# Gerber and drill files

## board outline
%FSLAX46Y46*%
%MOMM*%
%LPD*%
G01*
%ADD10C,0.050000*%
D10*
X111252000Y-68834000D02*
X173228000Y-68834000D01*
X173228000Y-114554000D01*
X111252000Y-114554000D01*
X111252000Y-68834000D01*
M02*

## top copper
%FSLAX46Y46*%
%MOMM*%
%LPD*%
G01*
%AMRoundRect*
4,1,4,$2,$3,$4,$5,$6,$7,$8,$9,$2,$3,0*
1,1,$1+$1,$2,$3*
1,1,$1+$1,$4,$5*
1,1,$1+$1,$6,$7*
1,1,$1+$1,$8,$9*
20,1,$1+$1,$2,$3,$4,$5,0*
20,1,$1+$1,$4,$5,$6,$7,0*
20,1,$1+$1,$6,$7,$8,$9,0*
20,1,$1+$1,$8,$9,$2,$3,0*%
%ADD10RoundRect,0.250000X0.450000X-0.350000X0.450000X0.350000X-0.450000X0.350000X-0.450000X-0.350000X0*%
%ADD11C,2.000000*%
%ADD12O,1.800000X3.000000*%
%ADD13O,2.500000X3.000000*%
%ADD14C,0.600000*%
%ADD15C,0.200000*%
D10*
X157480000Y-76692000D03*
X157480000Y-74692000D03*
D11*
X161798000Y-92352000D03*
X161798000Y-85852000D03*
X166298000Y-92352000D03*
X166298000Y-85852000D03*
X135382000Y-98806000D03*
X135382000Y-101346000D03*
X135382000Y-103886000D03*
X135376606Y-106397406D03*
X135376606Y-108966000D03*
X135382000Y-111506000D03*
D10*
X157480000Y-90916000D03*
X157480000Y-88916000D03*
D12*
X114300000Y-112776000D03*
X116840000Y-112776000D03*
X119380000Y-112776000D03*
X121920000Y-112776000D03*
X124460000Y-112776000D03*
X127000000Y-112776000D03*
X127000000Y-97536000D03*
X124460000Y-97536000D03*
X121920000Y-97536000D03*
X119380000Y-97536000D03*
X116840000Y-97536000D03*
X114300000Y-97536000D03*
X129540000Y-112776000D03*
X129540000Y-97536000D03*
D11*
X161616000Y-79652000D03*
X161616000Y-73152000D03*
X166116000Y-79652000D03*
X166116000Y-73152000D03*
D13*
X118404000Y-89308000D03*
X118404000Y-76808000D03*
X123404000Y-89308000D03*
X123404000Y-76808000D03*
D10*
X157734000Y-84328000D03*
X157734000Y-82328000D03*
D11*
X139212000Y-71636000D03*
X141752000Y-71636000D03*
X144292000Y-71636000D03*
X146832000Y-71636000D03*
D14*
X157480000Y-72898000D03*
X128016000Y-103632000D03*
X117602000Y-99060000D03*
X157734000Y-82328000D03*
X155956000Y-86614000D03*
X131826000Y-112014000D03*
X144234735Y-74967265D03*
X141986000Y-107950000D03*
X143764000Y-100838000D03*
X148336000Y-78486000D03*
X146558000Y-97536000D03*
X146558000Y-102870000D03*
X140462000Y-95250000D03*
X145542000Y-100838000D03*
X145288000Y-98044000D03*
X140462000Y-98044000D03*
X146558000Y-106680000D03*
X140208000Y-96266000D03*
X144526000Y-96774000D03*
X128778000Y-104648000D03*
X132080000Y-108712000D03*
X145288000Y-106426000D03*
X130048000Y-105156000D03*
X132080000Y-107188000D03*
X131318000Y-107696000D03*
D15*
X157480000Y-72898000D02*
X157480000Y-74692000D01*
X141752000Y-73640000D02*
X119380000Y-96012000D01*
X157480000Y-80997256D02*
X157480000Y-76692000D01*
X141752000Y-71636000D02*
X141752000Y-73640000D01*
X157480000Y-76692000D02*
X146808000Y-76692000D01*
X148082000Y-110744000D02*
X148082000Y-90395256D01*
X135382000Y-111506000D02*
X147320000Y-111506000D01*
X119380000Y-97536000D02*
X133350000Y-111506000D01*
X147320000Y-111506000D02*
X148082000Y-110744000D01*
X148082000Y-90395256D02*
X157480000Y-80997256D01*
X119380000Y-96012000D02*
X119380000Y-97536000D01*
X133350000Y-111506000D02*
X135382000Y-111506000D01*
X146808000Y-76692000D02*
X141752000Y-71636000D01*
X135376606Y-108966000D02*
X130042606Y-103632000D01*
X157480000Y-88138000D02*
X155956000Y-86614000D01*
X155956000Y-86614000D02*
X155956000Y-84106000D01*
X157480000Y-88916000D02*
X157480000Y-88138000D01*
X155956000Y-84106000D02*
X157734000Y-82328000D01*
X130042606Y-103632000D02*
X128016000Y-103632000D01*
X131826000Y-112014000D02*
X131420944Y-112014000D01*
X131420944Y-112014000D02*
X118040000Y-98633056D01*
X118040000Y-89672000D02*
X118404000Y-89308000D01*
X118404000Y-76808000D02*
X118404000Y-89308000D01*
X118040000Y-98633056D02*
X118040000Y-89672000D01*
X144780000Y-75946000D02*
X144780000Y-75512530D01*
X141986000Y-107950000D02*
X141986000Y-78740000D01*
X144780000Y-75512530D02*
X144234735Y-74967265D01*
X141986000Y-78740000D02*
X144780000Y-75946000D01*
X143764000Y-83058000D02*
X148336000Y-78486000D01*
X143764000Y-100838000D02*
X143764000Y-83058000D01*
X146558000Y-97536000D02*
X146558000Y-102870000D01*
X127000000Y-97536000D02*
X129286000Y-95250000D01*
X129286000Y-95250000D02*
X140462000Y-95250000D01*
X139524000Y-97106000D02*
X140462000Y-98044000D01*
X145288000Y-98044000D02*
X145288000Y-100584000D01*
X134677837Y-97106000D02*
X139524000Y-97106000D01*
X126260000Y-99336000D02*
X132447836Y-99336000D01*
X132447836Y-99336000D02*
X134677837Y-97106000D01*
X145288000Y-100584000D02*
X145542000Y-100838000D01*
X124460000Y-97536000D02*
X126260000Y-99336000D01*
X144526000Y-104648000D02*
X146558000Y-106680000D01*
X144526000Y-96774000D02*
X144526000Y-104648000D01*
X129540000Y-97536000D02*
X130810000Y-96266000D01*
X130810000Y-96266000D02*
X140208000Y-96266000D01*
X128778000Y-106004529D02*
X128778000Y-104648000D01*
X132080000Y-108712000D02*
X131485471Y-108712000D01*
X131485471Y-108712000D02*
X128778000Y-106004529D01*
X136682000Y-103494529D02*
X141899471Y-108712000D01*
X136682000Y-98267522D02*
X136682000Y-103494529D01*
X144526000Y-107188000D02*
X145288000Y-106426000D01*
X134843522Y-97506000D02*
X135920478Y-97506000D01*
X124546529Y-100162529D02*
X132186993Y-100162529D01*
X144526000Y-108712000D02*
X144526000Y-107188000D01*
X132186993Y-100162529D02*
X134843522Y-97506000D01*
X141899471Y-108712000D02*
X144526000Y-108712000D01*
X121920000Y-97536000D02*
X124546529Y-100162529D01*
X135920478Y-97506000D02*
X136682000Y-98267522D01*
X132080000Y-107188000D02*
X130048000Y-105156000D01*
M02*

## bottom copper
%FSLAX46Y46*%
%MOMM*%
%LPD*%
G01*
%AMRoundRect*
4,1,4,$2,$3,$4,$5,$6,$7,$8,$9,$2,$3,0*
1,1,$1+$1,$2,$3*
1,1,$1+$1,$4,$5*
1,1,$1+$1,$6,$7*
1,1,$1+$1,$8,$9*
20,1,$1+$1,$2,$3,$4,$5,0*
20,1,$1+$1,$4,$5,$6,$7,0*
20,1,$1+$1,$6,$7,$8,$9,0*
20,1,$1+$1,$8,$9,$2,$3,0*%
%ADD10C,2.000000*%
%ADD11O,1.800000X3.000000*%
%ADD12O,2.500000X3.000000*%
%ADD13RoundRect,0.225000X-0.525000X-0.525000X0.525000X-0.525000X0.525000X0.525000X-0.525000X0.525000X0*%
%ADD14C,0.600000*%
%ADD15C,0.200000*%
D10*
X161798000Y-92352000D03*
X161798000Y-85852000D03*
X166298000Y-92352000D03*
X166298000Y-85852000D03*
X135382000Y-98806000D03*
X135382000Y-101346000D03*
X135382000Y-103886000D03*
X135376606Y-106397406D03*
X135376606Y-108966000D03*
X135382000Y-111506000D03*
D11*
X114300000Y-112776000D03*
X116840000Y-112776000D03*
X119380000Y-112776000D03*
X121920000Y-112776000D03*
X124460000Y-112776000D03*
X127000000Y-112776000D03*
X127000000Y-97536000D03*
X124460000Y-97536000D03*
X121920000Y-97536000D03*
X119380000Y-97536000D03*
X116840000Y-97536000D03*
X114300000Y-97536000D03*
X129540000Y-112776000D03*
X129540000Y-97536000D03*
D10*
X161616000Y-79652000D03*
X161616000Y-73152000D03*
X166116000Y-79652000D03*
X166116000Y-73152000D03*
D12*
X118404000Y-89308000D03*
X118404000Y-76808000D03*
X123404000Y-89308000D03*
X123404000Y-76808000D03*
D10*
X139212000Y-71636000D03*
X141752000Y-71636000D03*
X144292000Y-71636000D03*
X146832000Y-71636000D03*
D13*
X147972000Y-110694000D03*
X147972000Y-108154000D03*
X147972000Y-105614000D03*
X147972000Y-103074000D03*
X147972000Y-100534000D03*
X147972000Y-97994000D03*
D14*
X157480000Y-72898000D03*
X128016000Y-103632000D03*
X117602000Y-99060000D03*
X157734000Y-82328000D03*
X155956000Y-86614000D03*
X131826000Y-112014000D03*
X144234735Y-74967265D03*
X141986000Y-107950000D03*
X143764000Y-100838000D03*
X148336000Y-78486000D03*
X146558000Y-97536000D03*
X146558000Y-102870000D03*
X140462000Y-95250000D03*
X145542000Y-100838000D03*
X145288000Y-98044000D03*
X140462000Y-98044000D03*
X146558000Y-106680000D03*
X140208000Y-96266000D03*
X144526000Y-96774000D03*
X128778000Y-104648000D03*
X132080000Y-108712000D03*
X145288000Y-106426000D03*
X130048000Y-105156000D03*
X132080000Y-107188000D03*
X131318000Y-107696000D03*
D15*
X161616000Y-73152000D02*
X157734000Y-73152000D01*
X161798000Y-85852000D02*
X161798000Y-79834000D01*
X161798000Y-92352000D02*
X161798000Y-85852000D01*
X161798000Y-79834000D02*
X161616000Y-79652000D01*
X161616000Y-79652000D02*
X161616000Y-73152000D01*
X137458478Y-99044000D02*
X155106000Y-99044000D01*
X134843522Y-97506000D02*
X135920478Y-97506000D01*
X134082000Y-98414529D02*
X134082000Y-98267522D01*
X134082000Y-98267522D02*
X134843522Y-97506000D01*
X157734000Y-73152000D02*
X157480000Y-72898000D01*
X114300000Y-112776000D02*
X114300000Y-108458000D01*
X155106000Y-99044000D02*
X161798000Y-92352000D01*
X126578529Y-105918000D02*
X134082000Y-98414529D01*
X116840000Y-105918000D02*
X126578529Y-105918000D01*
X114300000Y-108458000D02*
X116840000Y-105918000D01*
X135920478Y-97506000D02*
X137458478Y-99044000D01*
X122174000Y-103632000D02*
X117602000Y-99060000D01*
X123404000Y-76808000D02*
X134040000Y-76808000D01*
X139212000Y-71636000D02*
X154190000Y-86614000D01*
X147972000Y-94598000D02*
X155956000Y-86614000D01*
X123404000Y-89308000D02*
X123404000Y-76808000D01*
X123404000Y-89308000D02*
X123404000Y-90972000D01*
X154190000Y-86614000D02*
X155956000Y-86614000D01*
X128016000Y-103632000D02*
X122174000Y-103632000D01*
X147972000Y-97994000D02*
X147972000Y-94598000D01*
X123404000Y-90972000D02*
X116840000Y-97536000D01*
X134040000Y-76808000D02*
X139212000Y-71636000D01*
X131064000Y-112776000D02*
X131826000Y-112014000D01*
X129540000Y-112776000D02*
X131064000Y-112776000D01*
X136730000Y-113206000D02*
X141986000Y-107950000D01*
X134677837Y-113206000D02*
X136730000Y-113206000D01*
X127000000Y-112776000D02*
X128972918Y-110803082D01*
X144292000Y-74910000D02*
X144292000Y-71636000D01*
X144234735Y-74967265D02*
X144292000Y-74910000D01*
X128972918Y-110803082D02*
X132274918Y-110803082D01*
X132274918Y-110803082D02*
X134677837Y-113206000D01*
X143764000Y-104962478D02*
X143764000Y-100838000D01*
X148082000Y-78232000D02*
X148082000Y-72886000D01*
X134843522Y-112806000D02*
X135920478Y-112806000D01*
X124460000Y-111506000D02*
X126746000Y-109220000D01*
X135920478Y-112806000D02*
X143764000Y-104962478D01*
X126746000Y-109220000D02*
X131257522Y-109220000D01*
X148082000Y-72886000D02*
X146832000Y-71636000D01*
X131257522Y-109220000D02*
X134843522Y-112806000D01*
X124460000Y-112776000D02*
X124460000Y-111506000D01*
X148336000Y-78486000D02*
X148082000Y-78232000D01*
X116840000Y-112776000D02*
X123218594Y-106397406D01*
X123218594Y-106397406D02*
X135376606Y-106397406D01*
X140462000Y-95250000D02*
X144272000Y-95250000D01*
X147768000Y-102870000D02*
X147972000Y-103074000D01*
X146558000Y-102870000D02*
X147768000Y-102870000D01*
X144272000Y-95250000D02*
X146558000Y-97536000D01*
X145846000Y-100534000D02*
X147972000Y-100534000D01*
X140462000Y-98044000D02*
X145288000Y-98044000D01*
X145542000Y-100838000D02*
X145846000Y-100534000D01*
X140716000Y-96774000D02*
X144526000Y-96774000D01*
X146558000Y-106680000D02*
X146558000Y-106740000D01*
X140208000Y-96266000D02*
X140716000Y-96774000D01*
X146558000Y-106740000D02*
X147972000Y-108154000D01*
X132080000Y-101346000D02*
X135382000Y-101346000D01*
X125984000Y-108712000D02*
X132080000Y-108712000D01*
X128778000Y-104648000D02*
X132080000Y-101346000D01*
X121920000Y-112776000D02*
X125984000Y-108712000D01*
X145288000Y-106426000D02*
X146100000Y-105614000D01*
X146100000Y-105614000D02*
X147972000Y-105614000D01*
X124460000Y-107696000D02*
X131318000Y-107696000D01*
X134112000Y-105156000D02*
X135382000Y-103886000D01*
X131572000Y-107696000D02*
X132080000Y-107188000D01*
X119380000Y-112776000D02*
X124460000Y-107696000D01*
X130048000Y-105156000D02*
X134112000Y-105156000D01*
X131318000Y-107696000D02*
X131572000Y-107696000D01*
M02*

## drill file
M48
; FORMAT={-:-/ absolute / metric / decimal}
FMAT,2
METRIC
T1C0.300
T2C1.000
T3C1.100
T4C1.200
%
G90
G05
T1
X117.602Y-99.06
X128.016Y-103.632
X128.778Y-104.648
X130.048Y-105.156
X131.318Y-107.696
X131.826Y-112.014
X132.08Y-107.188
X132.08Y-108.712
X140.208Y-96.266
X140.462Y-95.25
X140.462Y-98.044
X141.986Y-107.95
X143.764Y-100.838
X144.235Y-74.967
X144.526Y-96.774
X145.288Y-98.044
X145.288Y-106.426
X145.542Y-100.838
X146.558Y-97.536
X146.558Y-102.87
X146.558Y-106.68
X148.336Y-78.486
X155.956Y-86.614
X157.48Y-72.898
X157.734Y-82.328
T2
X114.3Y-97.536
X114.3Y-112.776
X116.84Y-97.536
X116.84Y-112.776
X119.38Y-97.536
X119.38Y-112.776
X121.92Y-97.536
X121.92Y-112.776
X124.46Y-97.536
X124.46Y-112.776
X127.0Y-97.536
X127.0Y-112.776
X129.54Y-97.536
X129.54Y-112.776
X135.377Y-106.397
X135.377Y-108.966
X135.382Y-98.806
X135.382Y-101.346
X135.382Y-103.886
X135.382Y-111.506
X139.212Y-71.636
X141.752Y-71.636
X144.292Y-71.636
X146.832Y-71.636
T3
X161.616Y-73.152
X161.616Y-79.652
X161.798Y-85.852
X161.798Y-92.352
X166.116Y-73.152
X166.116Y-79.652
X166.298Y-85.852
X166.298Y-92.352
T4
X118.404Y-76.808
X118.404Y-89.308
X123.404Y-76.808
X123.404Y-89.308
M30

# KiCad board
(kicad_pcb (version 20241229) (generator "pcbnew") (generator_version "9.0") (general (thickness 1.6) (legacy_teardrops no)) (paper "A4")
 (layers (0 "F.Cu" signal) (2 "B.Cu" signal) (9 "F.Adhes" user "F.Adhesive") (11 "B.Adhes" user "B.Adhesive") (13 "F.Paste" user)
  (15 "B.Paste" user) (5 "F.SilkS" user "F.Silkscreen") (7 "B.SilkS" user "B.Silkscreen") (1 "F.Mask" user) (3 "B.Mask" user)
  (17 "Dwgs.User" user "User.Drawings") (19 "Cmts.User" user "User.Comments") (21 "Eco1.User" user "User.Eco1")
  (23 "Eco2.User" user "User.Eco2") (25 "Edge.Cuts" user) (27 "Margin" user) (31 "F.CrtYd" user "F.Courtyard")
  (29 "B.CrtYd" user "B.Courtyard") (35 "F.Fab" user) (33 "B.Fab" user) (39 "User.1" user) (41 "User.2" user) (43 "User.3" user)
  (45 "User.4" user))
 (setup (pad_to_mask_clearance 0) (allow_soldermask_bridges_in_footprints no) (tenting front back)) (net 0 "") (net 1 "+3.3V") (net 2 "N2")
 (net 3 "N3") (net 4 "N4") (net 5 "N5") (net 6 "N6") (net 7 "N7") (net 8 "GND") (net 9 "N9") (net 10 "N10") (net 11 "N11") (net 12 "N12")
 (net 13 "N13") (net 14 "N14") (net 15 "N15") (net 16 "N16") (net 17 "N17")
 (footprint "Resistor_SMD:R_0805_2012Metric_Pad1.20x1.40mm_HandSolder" (layer "F.Cu") (at 157.48 75.692 90)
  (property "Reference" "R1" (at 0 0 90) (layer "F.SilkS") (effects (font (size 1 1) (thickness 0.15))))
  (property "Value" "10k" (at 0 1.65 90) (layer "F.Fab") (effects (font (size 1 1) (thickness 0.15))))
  (pad "1" smd roundrect (at -1 0 90) (size 1.2 1.4) (layers "F.Cu" "F.Mask" "F.Paste") (roundrect_rratio 0.208333) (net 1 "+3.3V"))
  (pad "2" smd roundrect (at 1 0 90) (size 1.2 1.4) (layers "F.Cu" "F.Mask" "F.Paste") (roundrect_rratio 0.208333) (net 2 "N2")))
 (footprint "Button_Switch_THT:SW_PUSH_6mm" (layer "F.Cu") (at 161.798 92.352 90)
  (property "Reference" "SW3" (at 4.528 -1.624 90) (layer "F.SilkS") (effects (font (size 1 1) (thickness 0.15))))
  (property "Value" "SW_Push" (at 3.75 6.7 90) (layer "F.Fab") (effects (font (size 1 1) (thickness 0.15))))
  (pad "1" thru_hole circle (at 0 0 180) (size 2 2) (drill 1.1) (layers "*.Cu" "*.Mask") (remove_unused_layers no) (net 2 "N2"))
  (pad "1" thru_hole circle (at 6.5 0 180) (size 2 2) (drill 1.1) (layers "*.Cu" "*.Mask") (remove_unused_layers no) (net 2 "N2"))
  (pad "2" thru_hole circle (at 0 4.5 180) (size 2 2) (drill 1.1) (layers "*.Cu" "*.Mask") (remove_unused_layers no) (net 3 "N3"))
  (pad "2" thru_hole circle (at 6.5 4.5 180) (size 2 2) (drill 1.1) (layers "*.Cu" "*.Mask") (remove_unused_layers no) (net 3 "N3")))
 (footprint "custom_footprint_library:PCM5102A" (layer "F.Cu") (at 148.082 103.886)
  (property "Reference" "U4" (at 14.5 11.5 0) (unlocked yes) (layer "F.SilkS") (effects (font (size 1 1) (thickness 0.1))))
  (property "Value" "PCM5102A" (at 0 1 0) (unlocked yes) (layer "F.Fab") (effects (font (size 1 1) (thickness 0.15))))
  (pad "1" thru_hole circle (at -12.7 -5.08) (size 2 2) (drill 1) (layers "*.Cu" "*.Mask") (remove_unused_layers no) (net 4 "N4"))
  (pad "2" thru_hole circle (at -12.7 -2.54) (size 2 2) (drill 1) (layers "*.Cu" "*.Mask") (remove_unused_layers no) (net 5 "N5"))
  (pad "3" thru_hole circle (at -12.7 0) (size 2 2) (drill 1) (layers "*.Cu" "*.Mask") (remove_unused_layers no) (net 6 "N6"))
  (pad "4" thru_hole circle (at -12.705394 2.511406) (size 2 2) (drill 1) (layers "*.Cu" "*.Mask") (remove_unused_layers no) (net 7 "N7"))
  (pad "5" thru_hole circle (at -12.705394 5.08) (size 2 2) (drill 1) (layers "*.Cu" "*.Mask") (remove_unused_layers no) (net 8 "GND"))
  (pad "6" thru_hole circle (at -12.7 7.62) (size 2 2) (drill 1) (layers "*.Cu" "*.Mask") (remove_unused_layers no) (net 1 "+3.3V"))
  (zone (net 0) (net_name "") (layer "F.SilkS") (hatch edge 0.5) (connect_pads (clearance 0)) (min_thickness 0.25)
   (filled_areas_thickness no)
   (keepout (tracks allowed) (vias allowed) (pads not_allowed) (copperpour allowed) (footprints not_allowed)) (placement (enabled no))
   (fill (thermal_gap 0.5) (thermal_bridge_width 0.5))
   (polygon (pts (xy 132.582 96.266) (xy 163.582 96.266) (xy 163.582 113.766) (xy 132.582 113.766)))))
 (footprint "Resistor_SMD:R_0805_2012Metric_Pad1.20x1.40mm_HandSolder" (layer "F.Cu") (at 157.48 89.916 90)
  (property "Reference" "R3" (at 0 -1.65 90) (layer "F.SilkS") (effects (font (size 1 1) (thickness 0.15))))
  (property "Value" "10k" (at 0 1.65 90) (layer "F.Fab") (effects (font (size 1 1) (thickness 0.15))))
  (pad "1" smd roundrect (at -1 0 90) (size 1.2 1.4) (layers "F.Cu" "F.Mask" "F.Paste") (roundrect_rratio 0.208333) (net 3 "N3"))
  (pad "2" smd roundrect (at 1 0 90) (size 1.2 1.4) (layers "F.Cu" "F.Mask" "F.Paste") (roundrect_rratio 0.208333) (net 8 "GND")))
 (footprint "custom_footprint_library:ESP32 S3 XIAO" (layer "F.Cu") (at 121.92 105.156 90)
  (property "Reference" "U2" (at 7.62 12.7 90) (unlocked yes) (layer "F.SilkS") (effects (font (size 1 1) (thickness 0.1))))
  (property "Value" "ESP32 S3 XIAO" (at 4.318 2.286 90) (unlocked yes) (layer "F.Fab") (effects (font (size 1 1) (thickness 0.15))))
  (pad "1" thru_hole oval (at -7.62 -7.62 90) (size 3 1.8) (drill 1) (layers "*.Cu" "*.Mask") (remove_unused_layers no) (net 2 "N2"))
  (pad "2" thru_hole oval (at -7.62 -5.08 90) (size 3 1.8) (drill 1) (layers "*.Cu" "*.Mask") (remove_unused_layers no) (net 7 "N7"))
  (pad "3" thru_hole oval (at -7.62 -2.54 90) (size 3 1.8) (drill 1) (layers "*.Cu" "*.Mask") (remove_unused_layers no) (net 6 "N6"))
  (pad "4" thru_hole oval (at -7.62 0 90) (size 3 1.8) (drill 1) (layers "*.Cu" "*.Mask") (remove_unused_layers no) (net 5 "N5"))
  (pad "5" thru_hole oval (at -7.62 2.54 90) (size 3 1.8) (drill 1) (layers "*.Cu" "*.Mask") (remove_unused_layers no) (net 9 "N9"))
  (pad "6" thru_hole oval (at -7.62 5.08 90) (size 3 1.8) (drill 1) (layers "*.Cu" "*.Mask") (remove_unused_layers no) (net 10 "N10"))
  (pad "7" thru_hole oval (at 7.62 5.08 90) (size 3 1.8) (drill 1) (layers "*.Cu" "*.Mask") (remove_unused_layers no) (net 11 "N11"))
  (pad "8" thru_hole oval (at 7.62 2.54 90) (size 3 1.8) (drill 1) (layers "*.Cu" "*.Mask") (remove_unused_layers no) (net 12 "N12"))
  (pad "9" thru_hole oval (at 7.62 0 90) (size 3 1.8) (drill 1) (layers "*.Cu" "*.Mask") (remove_unused_layers no) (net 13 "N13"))
  (pad "10" thru_hole oval (at 7.62 -2.54 90) (size 3 1.8) (drill 1) (layers "*.Cu" "*.Mask") (remove_unused_layers no) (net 1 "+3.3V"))
  (pad "11" thru_hole oval (at 7.62 -5.08 90) (size 3 1.8) (drill 1) (layers "*.Cu" "*.Mask") (remove_unused_layers no) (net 8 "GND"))
  (pad "12" thru_hole oval (at 7.62 -7.62 90) (size 3 1.8) (drill 1) (layers "*.Cu" "*.Mask") (remove_unused_layers no) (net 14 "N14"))
  (pad "43" thru_hole oval (at -7.62 7.62 90) (size 3 1.8) (drill 1) (layers "*.Cu" "*.Mask") (remove_unused_layers no) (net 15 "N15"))
  (pad "44" thru_hole oval (at 7.62 7.62 90) (size 3 1.8) (drill 1) (layers "*.Cu" "*.Mask") (remove_unused_layers no) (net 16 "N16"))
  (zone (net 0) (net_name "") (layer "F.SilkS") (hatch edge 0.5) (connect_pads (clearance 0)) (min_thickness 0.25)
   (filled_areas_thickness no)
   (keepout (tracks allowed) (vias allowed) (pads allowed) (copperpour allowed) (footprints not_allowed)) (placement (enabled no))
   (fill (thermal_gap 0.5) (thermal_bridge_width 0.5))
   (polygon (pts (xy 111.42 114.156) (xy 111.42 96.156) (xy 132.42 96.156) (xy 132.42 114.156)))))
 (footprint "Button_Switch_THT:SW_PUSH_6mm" (layer "F.Cu") (at 161.616 79.652 90)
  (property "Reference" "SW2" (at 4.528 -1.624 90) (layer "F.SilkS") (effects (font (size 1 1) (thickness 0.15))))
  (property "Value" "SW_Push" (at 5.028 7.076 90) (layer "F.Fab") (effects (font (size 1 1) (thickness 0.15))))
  (pad "1" thru_hole circle (at 0 0 180) (size 2 2) (drill 1.1) (layers "*.Cu" "*.Mask") (remove_unused_layers no) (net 2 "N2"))
  (pad "1" thru_hole circle (at 6.5 0 180) (size 2 2) (drill 1.1) (layers "*.Cu" "*.Mask") (remove_unused_layers no) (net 2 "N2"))
  (pad "2" thru_hole circle (at 0 4.5 180) (size 2 2) (drill 1.1) (layers "*.Cu" "*.Mask") (remove_unused_layers no) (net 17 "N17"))
  (pad "2" thru_hole circle (at 6.5 4.5 180) (size 2 2) (drill 1.1) (layers "*.Cu" "*.Mask") (remove_unused_layers no) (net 17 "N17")))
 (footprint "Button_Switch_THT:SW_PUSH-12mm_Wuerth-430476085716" (layer "F.Cu") (at 118.404 89.308 90)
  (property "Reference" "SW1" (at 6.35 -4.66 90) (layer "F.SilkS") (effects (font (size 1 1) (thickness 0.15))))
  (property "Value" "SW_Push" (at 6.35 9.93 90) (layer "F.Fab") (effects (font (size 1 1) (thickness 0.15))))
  (pad "1" thru_hole oval (at 0 0 90) (size 3 2.5) (drill 1.2) (layers "*.Cu" "*.Mask") (remove_unused_layers no) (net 15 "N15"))
  (pad "1" thru_hole oval (at 12.5 0 90) (size 3 2.5) (drill 1.2) (layers "*.Cu" "*.Mask") (remove_unused_layers no) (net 15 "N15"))
  (pad "2" thru_hole oval (at 0 5 90) (size 3 2.5) (drill 1.2) (layers "*.Cu" "*.Mask") (remove_unused_layers no) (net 8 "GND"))
  (pad "2" thru_hole oval (at 12.5 5 90) (size 3 2.5) (drill 1.2) (layers "*.Cu" "*.Mask") (remove_unused_layers no) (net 8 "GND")))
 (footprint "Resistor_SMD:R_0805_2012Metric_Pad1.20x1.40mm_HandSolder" (layer "F.Cu") (at 157.734 83.328 90)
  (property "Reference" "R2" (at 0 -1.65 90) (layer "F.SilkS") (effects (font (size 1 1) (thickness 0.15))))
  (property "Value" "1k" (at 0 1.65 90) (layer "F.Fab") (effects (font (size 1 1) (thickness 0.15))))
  (pad "1" smd roundrect (at -1 0 90) (size 1.2 1.4) (layers "F.Cu" "F.Mask" "F.Paste") (roundrect_rratio 0.208333) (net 17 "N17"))
  (pad "2" smd roundrect (at 1 0 90) (size 1.2 1.4) (layers "F.Cu" "F.Mask" "F.Paste") (roundrect_rratio 0.208333) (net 8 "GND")))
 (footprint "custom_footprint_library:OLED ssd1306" (layer "F.Cu") (at 143.002 82.886)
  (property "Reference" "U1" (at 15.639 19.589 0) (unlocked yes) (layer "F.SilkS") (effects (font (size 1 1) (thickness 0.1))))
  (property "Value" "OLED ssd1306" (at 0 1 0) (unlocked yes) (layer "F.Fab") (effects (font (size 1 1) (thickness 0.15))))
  (pad "1" thru_hole circle (at -3.79 -11.25) (size 2 2) (drill 1) (layers "*.Cu" "*.Mask") (remove_unused_layers no) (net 8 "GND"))
  (pad "2" thru_hole circle (at -1.25 -11.25) (size 2 2) (drill 1) (layers "*.Cu" "*.Mask") (remove_unused_layers no) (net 1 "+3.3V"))
  (pad "3" thru_hole circle (at 1.29 -11.25) (size 2 2) (drill 1) (layers "*.Cu" "*.Mask") (remove_unused_layers no) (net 10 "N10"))
  (pad "4" thru_hole circle (at 3.83 -11.25) (size 2 2) (drill 1) (layers "*.Cu" "*.Mask") (remove_unused_layers no) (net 9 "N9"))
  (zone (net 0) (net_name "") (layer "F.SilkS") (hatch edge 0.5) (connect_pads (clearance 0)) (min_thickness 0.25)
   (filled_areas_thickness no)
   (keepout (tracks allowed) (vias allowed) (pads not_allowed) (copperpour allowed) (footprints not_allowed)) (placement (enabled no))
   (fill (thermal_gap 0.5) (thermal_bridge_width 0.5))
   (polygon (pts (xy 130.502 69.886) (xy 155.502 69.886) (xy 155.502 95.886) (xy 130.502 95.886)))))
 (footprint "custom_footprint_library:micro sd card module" (layer "B.Cu") (at 156.972 104.394)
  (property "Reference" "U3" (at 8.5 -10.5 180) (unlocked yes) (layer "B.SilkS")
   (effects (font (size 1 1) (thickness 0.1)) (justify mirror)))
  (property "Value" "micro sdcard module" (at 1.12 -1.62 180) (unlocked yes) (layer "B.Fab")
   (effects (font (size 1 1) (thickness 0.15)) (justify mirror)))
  (pad "1" smd roundrect (at -9 6.3) (size 1.5 1.5) (layers "B.Cu" "B.Mask" "B.Paste") (roundrect_rratio 0.15) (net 1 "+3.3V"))
  (pad "2" smd roundrect (at -9 3.76) (size 1.5 1.5) (layers "B.Cu" "B.Mask" "B.Paste") (roundrect_rratio 0.15) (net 16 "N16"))
  (pad "3" smd roundrect (at -9 1.22) (size 1.5 1.5) (layers "B.Cu" "B.Mask" "B.Paste") (roundrect_rratio 0.15) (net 13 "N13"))
  (pad "4" smd roundrect (at -9 -1.32) (size 1.5 1.5) (layers "B.Cu" "B.Mask" "B.Paste") (roundrect_rratio 0.15) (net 11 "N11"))
  (pad "5" smd roundrect (at -9 -3.86) (size 1.5 1.5) (layers "B.Cu" "B.Mask" "B.Paste") (roundrect_rratio 0.15) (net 12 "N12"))
  (pad "6" smd roundrect (at -9 -6.4) (size 1.5 1.5) (layers "B.Cu" "B.Mask" "B.Paste") (roundrect_rratio 0.15) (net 8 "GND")))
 (gr_rect (start 111.252 68.834) (end 173.228 114.554) (stroke (width 0.05) (type default)) (fill no) (layer "Edge.Cuts"))
 (segment (start 157.48 72.898) (end 157.48 74.692) (width 0.2) (layer "F.Cu") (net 2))
 (via (at 157.48 72.898) (size 0.6) (drill 0.3) (layers "F.Cu" "B.Cu") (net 2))
 (segment (start 161.616 73.152) (end 157.734 73.152) (width 0.2) (layer "B.Cu") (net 2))
 (segment (start 161.798 85.852) (end 161.798 79.834) (width 0.2) (layer "B.Cu") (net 2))
 (segment (start 161.798 92.352) (end 161.798 85.852) (width 0.2) (layer "B.Cu") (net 2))
 (segment (start 161.798 79.834) (end 161.616 79.652) (width 0.2) (layer "B.Cu") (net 2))
 (segment (start 161.616 79.652) (end 161.616 73.152) (width 0.2) (layer "B.Cu") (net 2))
 (segment (start 137.458478 99.044) (end 155.106 99.044) (width 0.2) (layer "B.Cu") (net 2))
 (segment (start 134.843522 97.506) (end 135.920478 97.506) (width 0.2) (layer "B.Cu") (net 2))
 (segment (start 134.082 98.414529) (end 134.082 98.267522) (width 0.2) (layer "B.Cu") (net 2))
 (segment (start 134.082 98.267522) (end 134.843522 97.506) (width 0.2) (layer "B.Cu") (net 2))
 (segment (start 157.734 73.152) (end 157.48 72.898) (width 0.2) (layer "B.Cu") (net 2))
 (segment (start 114.3 112.776) (end 114.3 108.458) (width 0.2) (layer "B.Cu") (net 2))
 (segment (start 155.106 99.044) (end 161.798 92.352) (width 0.2) (layer "B.Cu") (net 2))
 (segment (start 126.578529 105.918) (end 134.082 98.414529) (width 0.2) (layer "B.Cu") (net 2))
 (segment (start 116.84 105.918) (end 126.578529 105.918) (width 0.2) (layer "B.Cu") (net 2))
 (segment (start 114.3 108.458) (end 116.84 105.918) (width 0.2) (layer "B.Cu") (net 2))
 (segment (start 135.920478 97.506) (end 137.458478 99.044) (width 0.2) (layer "B.Cu") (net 2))
 (segment (start 141.752 73.64) (end 119.38 96.012) (width 0.2) (layer "F.Cu") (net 1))
 (segment (start 157.48 80.997256) (end 157.48 76.692) (width 0.2) (layer "F.Cu") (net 1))
 (segment (start 141.752 71.636) (end 141.752 73.64) (width 0.2) (layer "F.Cu") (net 1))
 (segment (start 157.48 76.692) (end 146.808 76.692) (width 0.2) (layer "F.Cu") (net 1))
 (segment (start 148.082 110.744) (end 148.082 90.395256) (width 0.2) (layer "F.Cu") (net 1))
 (segment (start 135.382 111.506) (end 147.32 111.506) (width 0.2) (layer "F.Cu") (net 1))
 (segment (start 119.38 97.536) (end 133.35 111.506) (width 0.2) (layer "F.Cu") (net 1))
 (segment (start 147.32 111.506) (end 148.082 110.744) (width 0.2) (layer "F.Cu") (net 1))
 (segment (start 148.082 90.395256) (end 157.48 80.997256) (width 0.2) (layer "F.Cu") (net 1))
 (segment (start 119.38 96.012) (end 119.38 97.536) (width 0.2) (layer "F.Cu") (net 1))
 (segment (start 133.35 111.506) (end 135.382 111.506) (width 0.2) (layer "F.Cu") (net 1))
 (segment (start 146.808 76.692) (end 141.752 71.636) (width 0.2) (layer "F.Cu") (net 1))
 (segment (start 135.376606 108.966) (end 130.042606 103.632) (width 0.2) (layer "F.Cu") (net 8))
 (segment (start 157.48 88.138) (end 155.956 86.614) (width 0.2) (layer "F.Cu") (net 8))
 (segment (start 155.956 86.614) (end 155.956 84.106) (width 0.2) (layer "F.Cu") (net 8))
 (segment (start 157.48 88.916) (end 157.48 88.138) (width 0.2) (layer "F.Cu") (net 8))
 (segment (start 155.956 84.106) (end 157.734 82.328) (width 0.2) (layer "F.Cu") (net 8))
 (segment (start 130.042606 103.632) (end 128.016 103.632) (width 0.2) (layer "F.Cu") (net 8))
 (via (at 128.016 103.632) (size 0.6) (drill 0.3) (layers "F.Cu" "B.Cu") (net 8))
 (via (at 117.602 99.06) (size 0.6) (drill 0.3) (layers "F.Cu" "B.Cu") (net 8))
 (via (at 157.734 82.328) (size 0.6) (drill 0.3) (layers "F.Cu" "B.Cu") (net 8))
 (via (at 155.956 86.614) (size 0.6) (drill 0.3) (layers "F.Cu" "B.Cu") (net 8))
 (segment (start 122.174 103.632) (end 117.602 99.06) (width 0.2) (layer "B.Cu") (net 8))
 (segment (start 123.404 76.808) (end 134.04 76.808) (width 0.2) (layer "B.Cu") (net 8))
 (segment (start 139.212 71.636) (end 154.19 86.614) (width 0.2) (layer "B.Cu") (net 8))
 (segment (start 147.972 94.598) (end 155.956 86.614) (width 0.2) (layer "B.Cu") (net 8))
 (segment (start 123.404 89.308) (end 123.404 76.808) (width 0.2) (layer "B.Cu") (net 8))
 (segment (start 123.404 89.308) (end 123.404 90.972) (width 0.2) (layer "B.Cu") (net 8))
 (segment (start 154.19 86.614) (end 155.956 86.614) (width 0.2) (layer "B.Cu") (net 8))
 (segment (start 128.016 103.632) (end 122.174 103.632) (width 0.2) (layer "B.Cu") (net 8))
 (segment (start 147.972 97.994) (end 147.972 94.598) (width 0.2) (layer "B.Cu") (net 8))
 (segment (start 123.404 90.972) (end 116.84 97.536) (width 0.2) (layer "B.Cu") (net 8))
 (segment (start 134.04 76.808) (end 139.212 71.636) (width 0.2) (layer "B.Cu") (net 8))
 (segment (start 131.826 112.014) (end 131.420944 112.014) (width 0.2) (layer "F.Cu") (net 15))
 (segment (start 131.420944 112.014) (end 118.04 98.633056) (width 0.2) (layer "F.Cu") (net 15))
 (segment (start 118.04 89.672) (end 118.404 89.308) (width 0.2) (layer "F.Cu") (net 15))
 (segment (start 118.404 76.808) (end 118.404 89.308) (width 0.2) (layer "F.Cu") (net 15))
 (segment (start 118.04 98.633056) (end 118.04 89.672) (width 0.2) (layer "F.Cu") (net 15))
 (via (at 131.826 112.014) (size 0.6) (drill 0.3) (layers "F.Cu" "B.Cu") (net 15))
 (segment (start 131.064 112.776) (end 131.826 112.014) (width 0.2) (layer "B.Cu") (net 15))
 (segment (start 129.54 112.776) (end 131.064 112.776) (width 0.2) (layer "B.Cu") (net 15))
 (segment (start 144.78 75.946) (end 144.78 75.51253) (width 0.2) (layer "F.Cu") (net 10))
 (segment (start 141.986 107.95) (end 141.986 78.74) (width 0.2) (layer "F.Cu") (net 10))
 (segment (start 144.78 75.51253) (end 144.234735 74.967265) (width 0.2) (layer "F.Cu") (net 10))
 (segment (start 141.986 78.74) (end 144.78 75.946) (width 0.2) (layer "F.Cu") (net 10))
 (via (at 144.234735 74.967265) (size 0.6) (drill 0.3) (layers "F.Cu" "B.Cu") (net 10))
 (via (at 141.986 107.95) (size 0.6) (drill 0.3) (layers "F.Cu" "B.Cu") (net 10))
 (segment (start 136.73 113.206) (end 141.986 107.95) (width 0.2) (layer "B.Cu") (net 10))
 (segment (start 134.677837 113.206) (end 136.73 113.206) (width 0.2) (layer "B.Cu") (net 10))
 (segment (start 127 112.776) (end 128.972918 110.803082) (width 0.2) (layer "B.Cu") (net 10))
 (segment (start 144.292 74.91) (end 144.292 71.636) (width 0.2) (layer "B.Cu") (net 10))
 (segment (start 144.234735 74.967265) (end 144.292 74.91) (width 0.2) (layer "B.Cu") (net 10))
 (segment (start 128.972918 110.803082) (end 132.274918 110.803082) (width 0.2) (layer "B.Cu") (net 10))
 (segment (start 132.274918 110.803082) (end 134.677837 113.206) (width 0.2) (layer "B.Cu") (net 10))
 (segment (start 143.764 83.058) (end 148.336 78.486) (width 0.2) (layer "F.Cu") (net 9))
 (segment (start 143.764 100.838) (end 143.764 83.058) (width 0.2) (layer "F.Cu") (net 9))
 (via (at 143.764 100.838) (size 0.6) (drill 0.3) (layers "F.Cu" "B.Cu") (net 9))
 (via (at 148.336 78.486) (size 0.6) (drill 0.3) (layers "F.Cu" "B.Cu") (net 9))
 (segment (start 143.764 104.962478) (end 143.764 100.838) (width 0.2) (layer "B.Cu") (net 9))
 (segment (start 148.082 78.232) (end 148.082 72.886) (width 0.2) (layer "B.Cu") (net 9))
 (segment (start 134.843522 112.806) (end 135.920478 112.806) (width 0.2) (layer "B.Cu") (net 9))
 (segment (start 124.46 111.506) (end 126.746 109.22) (width 0.2) (layer "B.Cu") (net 9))
 (segment (start 135.920478 112.806) (end 143.764 104.962478) (width 0.2) (layer "B.Cu") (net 9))
 (segment (start 126.746 109.22) (end 131.257522 109.22) (width 0.2) (layer "B.Cu") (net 9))
 (segment (start 148.082 72.886) (end 146.832 71.636) (width 0.2) (layer "B.Cu") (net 9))
 (segment (start 131.257522 109.22) (end 134.843522 112.806) (width 0.2) (layer "B.Cu") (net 9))
 (segment (start 124.46 112.776) (end 124.46 111.506) (width 0.2) (layer "B.Cu") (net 9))
 (segment (start 148.336 78.486) (end 148.082 78.232) (width 0.2) (layer "B.Cu") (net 9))
 (segment (start 116.84 112.776) (end 123.218594 106.397406) (width 0.2) (layer "B.Cu") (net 7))
 (segment (start 123.218594 106.397406) (end 135.376606 106.397406) (width 0.2) (layer "B.Cu") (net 7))
 (segment (start 146.558 97.536) (end 146.558 102.87) (width 0.2) (layer "F.Cu") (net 11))
 (segment (start 127 97.536) (end 129.286 95.25) (width 0.2) (layer "F.Cu") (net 11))
 (segment (start 129.286 95.25) (end 140.462 95.25) (width 0.2) (layer "F.Cu") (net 11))
 (via (at 146.558 97.536) (size 0.6) (drill 0.3) (layers "F.Cu" "B.Cu") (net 11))
 (via (at 146.558 102.87) (size 0.6) (drill 0.3) (layers "F.Cu" "B.Cu") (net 11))
 (via (at 140.462 95.25) (size 0.6) (drill 0.3) (layers "F.Cu" "B.Cu") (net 11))
 (segment (start 140.462 95.25) (end 144.272 95.25) (width 0.2) (layer "B.Cu") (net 11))
 (segment (start 147.768 102.87) (end 147.972 103.074) (width 0.2) (layer "B.Cu") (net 11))
 (segment (start 146.558 102.87) (end 147.768 102.87) (width 0.2) (layer "B.Cu") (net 11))
 (segment (start 144.272 95.25) (end 146.558 97.536) (width 0.2) (layer "B.Cu") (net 11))
 (segment (start 139.524 97.106) (end 140.462 98.044) (width 0.2) (layer "F.Cu") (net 12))
 (segment (start 145.288 98.044) (end 145.288 100.584) (width 0.2) (layer "F.Cu") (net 12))
 (segment (start 134.677837 97.106) (end 139.524 97.106) (width 0.2) (layer "F.Cu") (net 12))
 (segment (start 126.26 99.336) (end 132.447836 99.336) (width 0.2) (layer "F.Cu") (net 12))
 (segment (start 132.447836 99.336) (end 134.677837 97.106) (width 0.2) (layer "F.Cu") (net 12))
 (segment (start 145.288 100.584) (end 145.542 100.838) (width 0.2) (layer "F.Cu") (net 12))
 (segment (start 124.46 97.536) (end 126.26 99.336) (width 0.2) (layer "F.Cu") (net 12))
 (via (at 145.542 100.838) (size 0.6) (drill 0.3) (layers "F.Cu" "B.Cu") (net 12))
 (via (at 145.288 98.044) (size 0.6) (drill 0.3) (layers "F.Cu" "B.Cu") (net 12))
 (via (at 140.462 98.044) (size 0.6) (drill 0.3) (layers "F.Cu" "B.Cu") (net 12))
 (segment (start 145.846 100.534) (end 147.972 100.534) (width 0.2) (layer "B.Cu") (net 12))
 (segment (start 140.462 98.044) (end 145.288 98.044) (width 0.2) (layer "B.Cu") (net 12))
 (segment (start 145.542 100.838) (end 145.846 100.534) (width 0.2) (layer "B.Cu") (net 12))
 (segment (start 144.526 104.648) (end 146.558 106.68) (width 0.2) (layer "F.Cu") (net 16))
 (segment (start 144.526 96.774) (end 144.526 104.648) (width 0.2) (layer "F.Cu") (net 16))
 (segment (start 129.54 97.536) (end 130.81 96.266) (width 0.2) (layer "F.Cu") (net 16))
 (segment (start 130.81 96.266) (end 140.208 96.266) (width 0.2) (layer "F.Cu") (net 16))
 (via (at 146.558 106.68) (size 0.6) (drill 0.3) (layers "F.Cu" "B.Cu") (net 16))
 (via (at 140.208 96.266) (size 0.6) (drill 0.3) (layers "F.Cu" "B.Cu") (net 16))
 (via (at 144.526 96.774) (size 0.6) (drill 0.3) (layers "F.Cu" "B.Cu") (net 16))
 (segment (start 140.716 96.774) (end 144.526 96.774) (width 0.2) (layer "B.Cu") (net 16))
 (segment (start 146.558 106.68) (end 146.558 106.74) (width 0.2) (layer "B.Cu") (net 16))
 (segment (start 140.208 96.266) (end 140.716 96.774) (width 0.2) (layer "B.Cu") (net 16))
 (segment (start 146.558 106.74) (end 147.972 108.154) (width 0.2) (layer "B.Cu") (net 16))
 (segment (start 128.778 106.004529) (end 128.778 104.648) (width 0.2) (layer "F.Cu") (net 5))
 (segment (start 132.08 108.712) (end 131.485471 108.712) (width 0.2) (layer "F.Cu") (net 5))
 (segment (start 131.485471 108.712) (end 128.778 106.004529) (width 0.2) (layer "F.Cu") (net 5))
 (via (at 128.778 104.648) (size 0.6) (drill 0.3) (layers "F.Cu" "B.Cu") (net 5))
 (via (at 132.08 108.712) (size 0.6) (drill 0.3) (layers "F.Cu" "B.Cu") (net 5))
 (segment (start 132.08 101.346) (end 135.382 101.346) (width 0.2) (layer "B.Cu") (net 5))
 (segment (start 125.984 108.712) (end 132.08 108.712) (width 0.2) (layer "B.Cu") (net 5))
 (segment (start 128.778 104.648) (end 132.08 101.346) (width 0.2) (layer "B.Cu") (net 5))
 (segment (start 121.92 112.776) (end 125.984 108.712) (width 0.2) (layer "B.Cu") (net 5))
 (segment (start 136.682 103.494529) (end 141.899471 108.712) (width 0.2) (layer "F.Cu") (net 13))
 (segment (start 136.682 98.267522) (end 136.682 103.494529) (width 0.2) (layer "F.Cu") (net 13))
 (segment (start 144.526 107.188) (end 145.288 106.426) (width 0.2) (layer "F.Cu") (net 13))
 (segment (start 134.843522 97.506) (end 135.920478 97.506) (width 0.2) (layer "F.Cu") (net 13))
 (segment (start 124.546529 100.162529) (end 132.186993 100.162529) (width 0.2) (layer "F.Cu") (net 13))
 (segment (start 144.526 108.712) (end 144.526 107.188) (width 0.2) (layer "F.Cu") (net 13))
 (segment (start 132.186993 100.162529) (end 134.843522 97.506) (width 0.2) (layer "F.Cu") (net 13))
 (segment (start 141.899471 108.712) (end 144.526 108.712) (width 0.2) (layer "F.Cu") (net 13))
 (segment (start 121.92 97.536) (end 124.546529 100.162529) (width 0.2) (layer "F.Cu") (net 13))
 (segment (start 135.920478 97.506) (end 136.682 98.267522) (width 0.2) (layer "F.Cu") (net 13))
 (via (at 145.288 106.426) (size 0.6) (drill 0.3) (layers "F.Cu" "B.Cu") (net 13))
 (segment (start 145.288 106.426) (end 146.1 105.614) (width 0.2) (layer "B.Cu") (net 13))
 (segment (start 146.1 105.614) (end 147.972 105.614) (width 0.2) (layer "B.Cu") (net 13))
 (segment (start 132.08 107.188) (end 130.048 105.156) (width 0.2) (layer "F.Cu") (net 6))
 (via (at 130.048 105.156) (size 0.6) (drill 0.3) (layers "F.Cu" "B.Cu") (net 6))
 (via (at 132.08 107.188) (size 0.6) (drill 0.3) (layers "F.Cu" "B.Cu") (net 6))
 (via (at 131.318 107.696) (size 0.6) (drill 0.3) (layers "F.Cu" "B.Cu") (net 6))
 (segment (start 124.46 107.696) (end 131.318 107.696) (width 0.2) (layer "B.Cu") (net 6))
 (segment (start 134.112 105.156) (end 135.382 103.886) (width 0.2) (layer "B.Cu") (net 6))
 (segment (start 131.572 107.696) (end 132.08 107.188) (width 0.2) (layer "B.Cu") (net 6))
 (segment (start 119.38 112.776) (end 124.46 107.696) (width 0.2) (layer "B.Cu") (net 6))
 (segment (start 130.048 105.156) (end 134.112 105.156) (width 0.2) (layer "B.Cu") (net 6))
 (segment (start 131.318 107.696) (end 131.572 107.696) (width 0.2) (layer "B.Cu") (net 6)))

